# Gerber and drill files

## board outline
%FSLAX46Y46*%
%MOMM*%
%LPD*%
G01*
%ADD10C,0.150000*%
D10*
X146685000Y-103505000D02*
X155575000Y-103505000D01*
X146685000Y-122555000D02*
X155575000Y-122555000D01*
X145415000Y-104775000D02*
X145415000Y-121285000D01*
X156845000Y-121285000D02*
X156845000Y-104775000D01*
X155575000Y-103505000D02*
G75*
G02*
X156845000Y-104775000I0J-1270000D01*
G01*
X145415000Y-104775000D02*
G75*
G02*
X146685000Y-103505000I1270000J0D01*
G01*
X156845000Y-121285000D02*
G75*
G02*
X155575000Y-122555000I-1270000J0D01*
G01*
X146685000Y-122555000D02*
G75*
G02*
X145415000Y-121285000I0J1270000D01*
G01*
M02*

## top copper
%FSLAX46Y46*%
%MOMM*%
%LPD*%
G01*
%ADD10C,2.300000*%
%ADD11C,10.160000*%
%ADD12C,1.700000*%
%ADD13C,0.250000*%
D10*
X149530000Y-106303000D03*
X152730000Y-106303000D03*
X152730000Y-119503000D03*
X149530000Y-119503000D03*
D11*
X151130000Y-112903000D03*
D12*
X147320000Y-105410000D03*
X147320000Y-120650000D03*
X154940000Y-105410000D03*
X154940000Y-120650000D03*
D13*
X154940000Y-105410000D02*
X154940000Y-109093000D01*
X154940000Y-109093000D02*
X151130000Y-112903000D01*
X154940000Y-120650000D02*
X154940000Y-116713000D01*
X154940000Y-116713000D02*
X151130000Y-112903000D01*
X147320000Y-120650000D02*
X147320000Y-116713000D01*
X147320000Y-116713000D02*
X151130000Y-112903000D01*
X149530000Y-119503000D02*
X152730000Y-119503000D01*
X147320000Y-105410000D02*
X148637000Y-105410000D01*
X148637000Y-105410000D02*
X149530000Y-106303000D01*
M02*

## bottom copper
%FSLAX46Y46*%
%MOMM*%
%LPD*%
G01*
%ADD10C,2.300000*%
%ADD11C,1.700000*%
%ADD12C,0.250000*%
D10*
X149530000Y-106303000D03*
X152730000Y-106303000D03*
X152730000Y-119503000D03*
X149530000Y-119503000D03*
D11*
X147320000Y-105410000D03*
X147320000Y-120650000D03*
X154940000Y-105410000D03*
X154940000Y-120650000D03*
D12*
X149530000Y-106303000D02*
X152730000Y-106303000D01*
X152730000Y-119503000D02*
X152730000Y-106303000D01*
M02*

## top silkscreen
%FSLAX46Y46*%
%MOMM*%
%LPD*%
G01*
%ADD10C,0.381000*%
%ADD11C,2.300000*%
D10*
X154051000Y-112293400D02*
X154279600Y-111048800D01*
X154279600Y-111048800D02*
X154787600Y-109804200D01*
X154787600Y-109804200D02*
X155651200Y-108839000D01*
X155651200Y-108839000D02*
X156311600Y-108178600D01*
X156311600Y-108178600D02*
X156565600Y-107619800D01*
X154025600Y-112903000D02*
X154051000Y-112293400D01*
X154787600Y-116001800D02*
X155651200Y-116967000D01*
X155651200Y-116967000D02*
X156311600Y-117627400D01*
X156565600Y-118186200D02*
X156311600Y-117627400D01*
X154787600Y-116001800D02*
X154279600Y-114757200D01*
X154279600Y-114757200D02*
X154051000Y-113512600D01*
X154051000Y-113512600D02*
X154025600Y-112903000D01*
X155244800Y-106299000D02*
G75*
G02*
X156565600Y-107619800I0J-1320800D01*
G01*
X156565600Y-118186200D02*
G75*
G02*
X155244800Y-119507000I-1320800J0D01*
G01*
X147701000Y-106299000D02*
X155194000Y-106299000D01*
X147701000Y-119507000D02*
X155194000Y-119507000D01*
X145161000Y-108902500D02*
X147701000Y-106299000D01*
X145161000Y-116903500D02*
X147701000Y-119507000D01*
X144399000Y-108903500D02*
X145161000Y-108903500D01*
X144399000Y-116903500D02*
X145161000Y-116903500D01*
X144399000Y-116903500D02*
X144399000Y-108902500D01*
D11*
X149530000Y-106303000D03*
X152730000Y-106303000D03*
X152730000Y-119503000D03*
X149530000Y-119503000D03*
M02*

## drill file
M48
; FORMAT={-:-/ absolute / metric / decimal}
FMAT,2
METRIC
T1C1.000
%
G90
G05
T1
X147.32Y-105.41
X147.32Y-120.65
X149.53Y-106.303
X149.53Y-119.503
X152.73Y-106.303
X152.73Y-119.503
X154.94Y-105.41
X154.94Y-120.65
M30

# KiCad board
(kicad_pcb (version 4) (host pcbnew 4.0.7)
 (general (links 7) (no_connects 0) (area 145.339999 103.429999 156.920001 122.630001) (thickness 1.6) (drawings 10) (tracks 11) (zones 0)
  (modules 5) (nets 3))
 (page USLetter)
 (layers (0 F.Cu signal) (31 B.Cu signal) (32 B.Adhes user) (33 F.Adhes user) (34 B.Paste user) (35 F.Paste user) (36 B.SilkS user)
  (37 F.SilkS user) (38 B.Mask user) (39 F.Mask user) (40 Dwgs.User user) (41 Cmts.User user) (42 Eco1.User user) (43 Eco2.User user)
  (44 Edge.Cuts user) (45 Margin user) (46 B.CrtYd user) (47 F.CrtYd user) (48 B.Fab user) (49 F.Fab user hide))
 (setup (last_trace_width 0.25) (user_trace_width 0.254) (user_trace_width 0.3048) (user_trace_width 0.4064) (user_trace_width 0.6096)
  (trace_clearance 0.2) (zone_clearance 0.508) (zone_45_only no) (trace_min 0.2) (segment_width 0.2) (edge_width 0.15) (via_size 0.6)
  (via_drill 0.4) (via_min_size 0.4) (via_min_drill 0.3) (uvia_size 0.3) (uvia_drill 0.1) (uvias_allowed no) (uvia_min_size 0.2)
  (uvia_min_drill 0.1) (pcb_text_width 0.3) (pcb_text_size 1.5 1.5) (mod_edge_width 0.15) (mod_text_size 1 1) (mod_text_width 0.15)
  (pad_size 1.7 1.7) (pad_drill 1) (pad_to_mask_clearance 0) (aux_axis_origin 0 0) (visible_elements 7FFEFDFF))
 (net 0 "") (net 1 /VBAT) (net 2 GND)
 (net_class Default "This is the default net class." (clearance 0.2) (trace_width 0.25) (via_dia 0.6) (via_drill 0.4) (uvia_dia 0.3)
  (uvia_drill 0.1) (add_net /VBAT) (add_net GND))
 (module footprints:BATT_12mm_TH (layer F.Cu) (at 151.13 112.903 90)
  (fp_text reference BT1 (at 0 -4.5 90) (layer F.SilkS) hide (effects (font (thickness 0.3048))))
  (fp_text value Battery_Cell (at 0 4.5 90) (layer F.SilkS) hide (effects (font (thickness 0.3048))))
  (fp_line (start 0.6096 2.921) (end 1.8542 3.1496) (layer F.SilkS) (width 0.381))
  (fp_line (start 1.8542 3.1496) (end 3.0988 3.6576) (layer F.SilkS) (width 0.381))
  (fp_line (start 3.0988 3.6576) (end 4.064 4.5212) (layer F.SilkS) (width 0.381))
  (fp_line (start 4.064 4.5212) (end 4.7244 5.1816) (layer F.SilkS) (width 0.381))
  (fp_line (start 4.7244 5.1816) (end 5.2832 5.4356) (layer F.SilkS) (width 0.381))
  (fp_line (start 0 2.8956) (end 0.6096 2.921) (layer F.SilkS) (width 0.381))
  (fp_line (start -3.0988 3.6576) (end -4.064 4.5212) (layer F.SilkS) (width 0.381))
  (fp_line (start -4.064 4.5212) (end -4.7244 5.1816) (layer F.SilkS) (width 0.381))
  (fp_line (start -5.2832 5.4356) (end -4.7244 5.1816) (layer F.SilkS) (width 0.381))
  (fp_line (start -3.0988 3.6576) (end -1.8542 3.1496) (layer F.SilkS) (width 0.381))
  (fp_line (start -1.8542 3.1496) (end -0.6096 2.921) (layer F.SilkS) (width 0.381))
  (fp_line (start -0.6096 2.921) (end 0 2.8956) (layer F.SilkS) (width 0.381))
  (fp_arc (start 5.2832 4.1148) (end 6.604 4.1148) (angle 90) (layer F.SilkS) (width 0.381))
  (fp_arc (start -5.2832 4.1148) (end -5.2832 5.4356) (angle 90) (layer F.SilkS) (width 0.381))
  (fp_line (start 6.604 -3.429) (end 6.604 4.064) (layer F.SilkS) (width 0.381))
  (fp_line (start -6.604 -3.429) (end -6.604 4.064) (layer F.SilkS) (width 0.381))
  (fp_line (start 4.0005 -5.969) (end 6.604 -3.429) (layer F.SilkS) (width 0.381))
  (fp_line (start -4.0005 -5.969) (end -6.604 -3.429) (layer F.SilkS) (width 0.381))
  (fp_line (start 3.9995 -6.731) (end 3.9995 -5.969) (layer F.SilkS) (width 0.381))
  (fp_line (start -4.0005 -6.731) (end -4.0005 -5.969) (layer F.SilkS) (width 0.381))
  (fp_line (start -4.0005 -6.731) (end 4.0005 -6.731) (layer F.SilkS) (width 0.381))
  (pad 1 thru_hole circle (at 6.6 -1.6 90) (size 2.3 2.3) (drill 1) (layers *.Cu *.Mask F.SilkS) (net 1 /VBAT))
  (pad 1 thru_hole circle (at 6.6 1.6 90) (size 2.3 2.3) (drill 1) (layers *.Cu *.Mask F.SilkS) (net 1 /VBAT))
  (pad 1 thru_hole circle (at -6.6 1.6 90) (size 2.3 2.3) (drill 1) (layers *.Cu *.Mask F.SilkS) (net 1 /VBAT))
  (pad 1 thru_hole circle (at -6.6 -1.6 90) (size 2.3 2.3) (drill 1) (layers *.Cu *.Mask F.SilkS) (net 1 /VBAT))
  (pad 2 smd circle (at 0 0 90) (size 10.16 10.16) (layers F.Cu F.Paste F.Mask) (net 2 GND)))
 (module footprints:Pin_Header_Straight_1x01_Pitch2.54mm (layer F.Cu) (at 147.32 105.41)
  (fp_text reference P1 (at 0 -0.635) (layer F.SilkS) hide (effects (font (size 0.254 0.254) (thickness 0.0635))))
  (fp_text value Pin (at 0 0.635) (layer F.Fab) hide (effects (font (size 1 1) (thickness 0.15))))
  (pad 1 thru_hole circle (at 0 0) (size 1.7 1.7) (drill 1) (layers *.Cu *.Mask) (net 1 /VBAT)))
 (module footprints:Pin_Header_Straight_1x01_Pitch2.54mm (layer F.Cu) (at 147.32 120.65)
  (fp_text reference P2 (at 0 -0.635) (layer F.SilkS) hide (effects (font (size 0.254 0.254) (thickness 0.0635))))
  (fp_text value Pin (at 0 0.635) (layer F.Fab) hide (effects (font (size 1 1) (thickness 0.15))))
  (pad 1 thru_hole circle (at 0 0) (size 1.7 1.7) (drill 1) (layers *.Cu *.Mask) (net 2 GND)))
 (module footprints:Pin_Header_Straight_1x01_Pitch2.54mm (layer F.Cu) (at 154.94 105.41)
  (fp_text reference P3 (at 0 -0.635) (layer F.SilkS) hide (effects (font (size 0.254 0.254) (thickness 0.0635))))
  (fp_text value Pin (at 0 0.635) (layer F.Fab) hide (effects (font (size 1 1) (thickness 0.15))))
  (pad 1 thru_hole circle (at 0 0) (size 1.7 1.7) (drill 1) (layers *.Cu *.Mask) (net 2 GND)))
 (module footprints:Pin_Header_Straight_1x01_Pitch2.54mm (layer F.Cu) (at 154.94 120.65)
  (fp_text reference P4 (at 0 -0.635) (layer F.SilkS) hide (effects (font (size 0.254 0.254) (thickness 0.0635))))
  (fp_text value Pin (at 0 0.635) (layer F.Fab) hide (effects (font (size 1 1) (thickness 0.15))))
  (pad 1 thru_hole circle (at 0 0) (size 1.7 1.7) (drill 1) (layers *.Cu *.Mask) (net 2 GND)))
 (gr_line (start 146.685 103.505) (end 155.575 103.505) (angle 90) (layer Edge.Cuts) (width 0.15))
 (gr_line (start 146.685 122.555) (end 155.575 122.555) (angle 90) (layer Edge.Cuts) (width 0.15))
 (gr_line (start 145.415 104.775) (end 145.415 121.285) (angle 90) (layer Edge.Cuts) (width 0.15))
 (gr_line (start 156.845 121.285) (end 156.845 104.775) (angle 90) (layer Edge.Cuts) (width 0.15))
 (gr_arc (start 155.575 104.775) (end 155.575 103.505) (angle 90) (layer Edge.Cuts) (width 0.15))
 (gr_arc (start 146.685 104.775) (end 145.415 104.775) (angle 90) (layer Edge.Cuts) (width 0.15))
 (gr_arc (start 155.575 121.285) (end 156.845 121.285) (angle 90) (layer Edge.Cuts) (width 0.15))
 (gr_arc (start 146.685 121.285) (end 146.685 122.555) (angle 90) (layer Edge.Cuts) (width 0.15))
 (segment (start 154.94 105.41) (end 154.94 109.093) (width 0.25) (layer F.Cu) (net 2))
 (segment (start 154.94 109.093) (end 151.13 112.903) (width 0.25) (layer F.Cu) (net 2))
 (segment (start 154.94 120.65) (end 154.94 116.713) (width 0.25) (layer F.Cu) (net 2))
 (segment (start 154.94 116.713) (end 151.13 112.903) (width 0.25) (layer F.Cu) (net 2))
 (segment (start 147.32 120.65) (end 147.32 116.713) (width 0.25) (layer F.Cu) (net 2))
 (segment (start 147.32 116.713) (end 151.13 112.903) (width 0.25) (layer F.Cu) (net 2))
 (segment (start 149.53 106.303) (end 152.73 106.303) (width 0.25) (layer B.Cu) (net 1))
 (segment (start 152.73 119.503) (end 152.73 106.303) (width 0.25) (layer B.Cu) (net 1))
 (segment (start 149.53 119.503) (end 152.73 119.503) (width 0.25) (layer F.Cu) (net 1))
 (segment (start 147.32 105.41) (end 148.637 105.41) (width 0.25) (layer F.Cu) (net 1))
 (segment (start 148.637 105.41) (end 149.53 106.303) (width 0.25) (layer F.Cu) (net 1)))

